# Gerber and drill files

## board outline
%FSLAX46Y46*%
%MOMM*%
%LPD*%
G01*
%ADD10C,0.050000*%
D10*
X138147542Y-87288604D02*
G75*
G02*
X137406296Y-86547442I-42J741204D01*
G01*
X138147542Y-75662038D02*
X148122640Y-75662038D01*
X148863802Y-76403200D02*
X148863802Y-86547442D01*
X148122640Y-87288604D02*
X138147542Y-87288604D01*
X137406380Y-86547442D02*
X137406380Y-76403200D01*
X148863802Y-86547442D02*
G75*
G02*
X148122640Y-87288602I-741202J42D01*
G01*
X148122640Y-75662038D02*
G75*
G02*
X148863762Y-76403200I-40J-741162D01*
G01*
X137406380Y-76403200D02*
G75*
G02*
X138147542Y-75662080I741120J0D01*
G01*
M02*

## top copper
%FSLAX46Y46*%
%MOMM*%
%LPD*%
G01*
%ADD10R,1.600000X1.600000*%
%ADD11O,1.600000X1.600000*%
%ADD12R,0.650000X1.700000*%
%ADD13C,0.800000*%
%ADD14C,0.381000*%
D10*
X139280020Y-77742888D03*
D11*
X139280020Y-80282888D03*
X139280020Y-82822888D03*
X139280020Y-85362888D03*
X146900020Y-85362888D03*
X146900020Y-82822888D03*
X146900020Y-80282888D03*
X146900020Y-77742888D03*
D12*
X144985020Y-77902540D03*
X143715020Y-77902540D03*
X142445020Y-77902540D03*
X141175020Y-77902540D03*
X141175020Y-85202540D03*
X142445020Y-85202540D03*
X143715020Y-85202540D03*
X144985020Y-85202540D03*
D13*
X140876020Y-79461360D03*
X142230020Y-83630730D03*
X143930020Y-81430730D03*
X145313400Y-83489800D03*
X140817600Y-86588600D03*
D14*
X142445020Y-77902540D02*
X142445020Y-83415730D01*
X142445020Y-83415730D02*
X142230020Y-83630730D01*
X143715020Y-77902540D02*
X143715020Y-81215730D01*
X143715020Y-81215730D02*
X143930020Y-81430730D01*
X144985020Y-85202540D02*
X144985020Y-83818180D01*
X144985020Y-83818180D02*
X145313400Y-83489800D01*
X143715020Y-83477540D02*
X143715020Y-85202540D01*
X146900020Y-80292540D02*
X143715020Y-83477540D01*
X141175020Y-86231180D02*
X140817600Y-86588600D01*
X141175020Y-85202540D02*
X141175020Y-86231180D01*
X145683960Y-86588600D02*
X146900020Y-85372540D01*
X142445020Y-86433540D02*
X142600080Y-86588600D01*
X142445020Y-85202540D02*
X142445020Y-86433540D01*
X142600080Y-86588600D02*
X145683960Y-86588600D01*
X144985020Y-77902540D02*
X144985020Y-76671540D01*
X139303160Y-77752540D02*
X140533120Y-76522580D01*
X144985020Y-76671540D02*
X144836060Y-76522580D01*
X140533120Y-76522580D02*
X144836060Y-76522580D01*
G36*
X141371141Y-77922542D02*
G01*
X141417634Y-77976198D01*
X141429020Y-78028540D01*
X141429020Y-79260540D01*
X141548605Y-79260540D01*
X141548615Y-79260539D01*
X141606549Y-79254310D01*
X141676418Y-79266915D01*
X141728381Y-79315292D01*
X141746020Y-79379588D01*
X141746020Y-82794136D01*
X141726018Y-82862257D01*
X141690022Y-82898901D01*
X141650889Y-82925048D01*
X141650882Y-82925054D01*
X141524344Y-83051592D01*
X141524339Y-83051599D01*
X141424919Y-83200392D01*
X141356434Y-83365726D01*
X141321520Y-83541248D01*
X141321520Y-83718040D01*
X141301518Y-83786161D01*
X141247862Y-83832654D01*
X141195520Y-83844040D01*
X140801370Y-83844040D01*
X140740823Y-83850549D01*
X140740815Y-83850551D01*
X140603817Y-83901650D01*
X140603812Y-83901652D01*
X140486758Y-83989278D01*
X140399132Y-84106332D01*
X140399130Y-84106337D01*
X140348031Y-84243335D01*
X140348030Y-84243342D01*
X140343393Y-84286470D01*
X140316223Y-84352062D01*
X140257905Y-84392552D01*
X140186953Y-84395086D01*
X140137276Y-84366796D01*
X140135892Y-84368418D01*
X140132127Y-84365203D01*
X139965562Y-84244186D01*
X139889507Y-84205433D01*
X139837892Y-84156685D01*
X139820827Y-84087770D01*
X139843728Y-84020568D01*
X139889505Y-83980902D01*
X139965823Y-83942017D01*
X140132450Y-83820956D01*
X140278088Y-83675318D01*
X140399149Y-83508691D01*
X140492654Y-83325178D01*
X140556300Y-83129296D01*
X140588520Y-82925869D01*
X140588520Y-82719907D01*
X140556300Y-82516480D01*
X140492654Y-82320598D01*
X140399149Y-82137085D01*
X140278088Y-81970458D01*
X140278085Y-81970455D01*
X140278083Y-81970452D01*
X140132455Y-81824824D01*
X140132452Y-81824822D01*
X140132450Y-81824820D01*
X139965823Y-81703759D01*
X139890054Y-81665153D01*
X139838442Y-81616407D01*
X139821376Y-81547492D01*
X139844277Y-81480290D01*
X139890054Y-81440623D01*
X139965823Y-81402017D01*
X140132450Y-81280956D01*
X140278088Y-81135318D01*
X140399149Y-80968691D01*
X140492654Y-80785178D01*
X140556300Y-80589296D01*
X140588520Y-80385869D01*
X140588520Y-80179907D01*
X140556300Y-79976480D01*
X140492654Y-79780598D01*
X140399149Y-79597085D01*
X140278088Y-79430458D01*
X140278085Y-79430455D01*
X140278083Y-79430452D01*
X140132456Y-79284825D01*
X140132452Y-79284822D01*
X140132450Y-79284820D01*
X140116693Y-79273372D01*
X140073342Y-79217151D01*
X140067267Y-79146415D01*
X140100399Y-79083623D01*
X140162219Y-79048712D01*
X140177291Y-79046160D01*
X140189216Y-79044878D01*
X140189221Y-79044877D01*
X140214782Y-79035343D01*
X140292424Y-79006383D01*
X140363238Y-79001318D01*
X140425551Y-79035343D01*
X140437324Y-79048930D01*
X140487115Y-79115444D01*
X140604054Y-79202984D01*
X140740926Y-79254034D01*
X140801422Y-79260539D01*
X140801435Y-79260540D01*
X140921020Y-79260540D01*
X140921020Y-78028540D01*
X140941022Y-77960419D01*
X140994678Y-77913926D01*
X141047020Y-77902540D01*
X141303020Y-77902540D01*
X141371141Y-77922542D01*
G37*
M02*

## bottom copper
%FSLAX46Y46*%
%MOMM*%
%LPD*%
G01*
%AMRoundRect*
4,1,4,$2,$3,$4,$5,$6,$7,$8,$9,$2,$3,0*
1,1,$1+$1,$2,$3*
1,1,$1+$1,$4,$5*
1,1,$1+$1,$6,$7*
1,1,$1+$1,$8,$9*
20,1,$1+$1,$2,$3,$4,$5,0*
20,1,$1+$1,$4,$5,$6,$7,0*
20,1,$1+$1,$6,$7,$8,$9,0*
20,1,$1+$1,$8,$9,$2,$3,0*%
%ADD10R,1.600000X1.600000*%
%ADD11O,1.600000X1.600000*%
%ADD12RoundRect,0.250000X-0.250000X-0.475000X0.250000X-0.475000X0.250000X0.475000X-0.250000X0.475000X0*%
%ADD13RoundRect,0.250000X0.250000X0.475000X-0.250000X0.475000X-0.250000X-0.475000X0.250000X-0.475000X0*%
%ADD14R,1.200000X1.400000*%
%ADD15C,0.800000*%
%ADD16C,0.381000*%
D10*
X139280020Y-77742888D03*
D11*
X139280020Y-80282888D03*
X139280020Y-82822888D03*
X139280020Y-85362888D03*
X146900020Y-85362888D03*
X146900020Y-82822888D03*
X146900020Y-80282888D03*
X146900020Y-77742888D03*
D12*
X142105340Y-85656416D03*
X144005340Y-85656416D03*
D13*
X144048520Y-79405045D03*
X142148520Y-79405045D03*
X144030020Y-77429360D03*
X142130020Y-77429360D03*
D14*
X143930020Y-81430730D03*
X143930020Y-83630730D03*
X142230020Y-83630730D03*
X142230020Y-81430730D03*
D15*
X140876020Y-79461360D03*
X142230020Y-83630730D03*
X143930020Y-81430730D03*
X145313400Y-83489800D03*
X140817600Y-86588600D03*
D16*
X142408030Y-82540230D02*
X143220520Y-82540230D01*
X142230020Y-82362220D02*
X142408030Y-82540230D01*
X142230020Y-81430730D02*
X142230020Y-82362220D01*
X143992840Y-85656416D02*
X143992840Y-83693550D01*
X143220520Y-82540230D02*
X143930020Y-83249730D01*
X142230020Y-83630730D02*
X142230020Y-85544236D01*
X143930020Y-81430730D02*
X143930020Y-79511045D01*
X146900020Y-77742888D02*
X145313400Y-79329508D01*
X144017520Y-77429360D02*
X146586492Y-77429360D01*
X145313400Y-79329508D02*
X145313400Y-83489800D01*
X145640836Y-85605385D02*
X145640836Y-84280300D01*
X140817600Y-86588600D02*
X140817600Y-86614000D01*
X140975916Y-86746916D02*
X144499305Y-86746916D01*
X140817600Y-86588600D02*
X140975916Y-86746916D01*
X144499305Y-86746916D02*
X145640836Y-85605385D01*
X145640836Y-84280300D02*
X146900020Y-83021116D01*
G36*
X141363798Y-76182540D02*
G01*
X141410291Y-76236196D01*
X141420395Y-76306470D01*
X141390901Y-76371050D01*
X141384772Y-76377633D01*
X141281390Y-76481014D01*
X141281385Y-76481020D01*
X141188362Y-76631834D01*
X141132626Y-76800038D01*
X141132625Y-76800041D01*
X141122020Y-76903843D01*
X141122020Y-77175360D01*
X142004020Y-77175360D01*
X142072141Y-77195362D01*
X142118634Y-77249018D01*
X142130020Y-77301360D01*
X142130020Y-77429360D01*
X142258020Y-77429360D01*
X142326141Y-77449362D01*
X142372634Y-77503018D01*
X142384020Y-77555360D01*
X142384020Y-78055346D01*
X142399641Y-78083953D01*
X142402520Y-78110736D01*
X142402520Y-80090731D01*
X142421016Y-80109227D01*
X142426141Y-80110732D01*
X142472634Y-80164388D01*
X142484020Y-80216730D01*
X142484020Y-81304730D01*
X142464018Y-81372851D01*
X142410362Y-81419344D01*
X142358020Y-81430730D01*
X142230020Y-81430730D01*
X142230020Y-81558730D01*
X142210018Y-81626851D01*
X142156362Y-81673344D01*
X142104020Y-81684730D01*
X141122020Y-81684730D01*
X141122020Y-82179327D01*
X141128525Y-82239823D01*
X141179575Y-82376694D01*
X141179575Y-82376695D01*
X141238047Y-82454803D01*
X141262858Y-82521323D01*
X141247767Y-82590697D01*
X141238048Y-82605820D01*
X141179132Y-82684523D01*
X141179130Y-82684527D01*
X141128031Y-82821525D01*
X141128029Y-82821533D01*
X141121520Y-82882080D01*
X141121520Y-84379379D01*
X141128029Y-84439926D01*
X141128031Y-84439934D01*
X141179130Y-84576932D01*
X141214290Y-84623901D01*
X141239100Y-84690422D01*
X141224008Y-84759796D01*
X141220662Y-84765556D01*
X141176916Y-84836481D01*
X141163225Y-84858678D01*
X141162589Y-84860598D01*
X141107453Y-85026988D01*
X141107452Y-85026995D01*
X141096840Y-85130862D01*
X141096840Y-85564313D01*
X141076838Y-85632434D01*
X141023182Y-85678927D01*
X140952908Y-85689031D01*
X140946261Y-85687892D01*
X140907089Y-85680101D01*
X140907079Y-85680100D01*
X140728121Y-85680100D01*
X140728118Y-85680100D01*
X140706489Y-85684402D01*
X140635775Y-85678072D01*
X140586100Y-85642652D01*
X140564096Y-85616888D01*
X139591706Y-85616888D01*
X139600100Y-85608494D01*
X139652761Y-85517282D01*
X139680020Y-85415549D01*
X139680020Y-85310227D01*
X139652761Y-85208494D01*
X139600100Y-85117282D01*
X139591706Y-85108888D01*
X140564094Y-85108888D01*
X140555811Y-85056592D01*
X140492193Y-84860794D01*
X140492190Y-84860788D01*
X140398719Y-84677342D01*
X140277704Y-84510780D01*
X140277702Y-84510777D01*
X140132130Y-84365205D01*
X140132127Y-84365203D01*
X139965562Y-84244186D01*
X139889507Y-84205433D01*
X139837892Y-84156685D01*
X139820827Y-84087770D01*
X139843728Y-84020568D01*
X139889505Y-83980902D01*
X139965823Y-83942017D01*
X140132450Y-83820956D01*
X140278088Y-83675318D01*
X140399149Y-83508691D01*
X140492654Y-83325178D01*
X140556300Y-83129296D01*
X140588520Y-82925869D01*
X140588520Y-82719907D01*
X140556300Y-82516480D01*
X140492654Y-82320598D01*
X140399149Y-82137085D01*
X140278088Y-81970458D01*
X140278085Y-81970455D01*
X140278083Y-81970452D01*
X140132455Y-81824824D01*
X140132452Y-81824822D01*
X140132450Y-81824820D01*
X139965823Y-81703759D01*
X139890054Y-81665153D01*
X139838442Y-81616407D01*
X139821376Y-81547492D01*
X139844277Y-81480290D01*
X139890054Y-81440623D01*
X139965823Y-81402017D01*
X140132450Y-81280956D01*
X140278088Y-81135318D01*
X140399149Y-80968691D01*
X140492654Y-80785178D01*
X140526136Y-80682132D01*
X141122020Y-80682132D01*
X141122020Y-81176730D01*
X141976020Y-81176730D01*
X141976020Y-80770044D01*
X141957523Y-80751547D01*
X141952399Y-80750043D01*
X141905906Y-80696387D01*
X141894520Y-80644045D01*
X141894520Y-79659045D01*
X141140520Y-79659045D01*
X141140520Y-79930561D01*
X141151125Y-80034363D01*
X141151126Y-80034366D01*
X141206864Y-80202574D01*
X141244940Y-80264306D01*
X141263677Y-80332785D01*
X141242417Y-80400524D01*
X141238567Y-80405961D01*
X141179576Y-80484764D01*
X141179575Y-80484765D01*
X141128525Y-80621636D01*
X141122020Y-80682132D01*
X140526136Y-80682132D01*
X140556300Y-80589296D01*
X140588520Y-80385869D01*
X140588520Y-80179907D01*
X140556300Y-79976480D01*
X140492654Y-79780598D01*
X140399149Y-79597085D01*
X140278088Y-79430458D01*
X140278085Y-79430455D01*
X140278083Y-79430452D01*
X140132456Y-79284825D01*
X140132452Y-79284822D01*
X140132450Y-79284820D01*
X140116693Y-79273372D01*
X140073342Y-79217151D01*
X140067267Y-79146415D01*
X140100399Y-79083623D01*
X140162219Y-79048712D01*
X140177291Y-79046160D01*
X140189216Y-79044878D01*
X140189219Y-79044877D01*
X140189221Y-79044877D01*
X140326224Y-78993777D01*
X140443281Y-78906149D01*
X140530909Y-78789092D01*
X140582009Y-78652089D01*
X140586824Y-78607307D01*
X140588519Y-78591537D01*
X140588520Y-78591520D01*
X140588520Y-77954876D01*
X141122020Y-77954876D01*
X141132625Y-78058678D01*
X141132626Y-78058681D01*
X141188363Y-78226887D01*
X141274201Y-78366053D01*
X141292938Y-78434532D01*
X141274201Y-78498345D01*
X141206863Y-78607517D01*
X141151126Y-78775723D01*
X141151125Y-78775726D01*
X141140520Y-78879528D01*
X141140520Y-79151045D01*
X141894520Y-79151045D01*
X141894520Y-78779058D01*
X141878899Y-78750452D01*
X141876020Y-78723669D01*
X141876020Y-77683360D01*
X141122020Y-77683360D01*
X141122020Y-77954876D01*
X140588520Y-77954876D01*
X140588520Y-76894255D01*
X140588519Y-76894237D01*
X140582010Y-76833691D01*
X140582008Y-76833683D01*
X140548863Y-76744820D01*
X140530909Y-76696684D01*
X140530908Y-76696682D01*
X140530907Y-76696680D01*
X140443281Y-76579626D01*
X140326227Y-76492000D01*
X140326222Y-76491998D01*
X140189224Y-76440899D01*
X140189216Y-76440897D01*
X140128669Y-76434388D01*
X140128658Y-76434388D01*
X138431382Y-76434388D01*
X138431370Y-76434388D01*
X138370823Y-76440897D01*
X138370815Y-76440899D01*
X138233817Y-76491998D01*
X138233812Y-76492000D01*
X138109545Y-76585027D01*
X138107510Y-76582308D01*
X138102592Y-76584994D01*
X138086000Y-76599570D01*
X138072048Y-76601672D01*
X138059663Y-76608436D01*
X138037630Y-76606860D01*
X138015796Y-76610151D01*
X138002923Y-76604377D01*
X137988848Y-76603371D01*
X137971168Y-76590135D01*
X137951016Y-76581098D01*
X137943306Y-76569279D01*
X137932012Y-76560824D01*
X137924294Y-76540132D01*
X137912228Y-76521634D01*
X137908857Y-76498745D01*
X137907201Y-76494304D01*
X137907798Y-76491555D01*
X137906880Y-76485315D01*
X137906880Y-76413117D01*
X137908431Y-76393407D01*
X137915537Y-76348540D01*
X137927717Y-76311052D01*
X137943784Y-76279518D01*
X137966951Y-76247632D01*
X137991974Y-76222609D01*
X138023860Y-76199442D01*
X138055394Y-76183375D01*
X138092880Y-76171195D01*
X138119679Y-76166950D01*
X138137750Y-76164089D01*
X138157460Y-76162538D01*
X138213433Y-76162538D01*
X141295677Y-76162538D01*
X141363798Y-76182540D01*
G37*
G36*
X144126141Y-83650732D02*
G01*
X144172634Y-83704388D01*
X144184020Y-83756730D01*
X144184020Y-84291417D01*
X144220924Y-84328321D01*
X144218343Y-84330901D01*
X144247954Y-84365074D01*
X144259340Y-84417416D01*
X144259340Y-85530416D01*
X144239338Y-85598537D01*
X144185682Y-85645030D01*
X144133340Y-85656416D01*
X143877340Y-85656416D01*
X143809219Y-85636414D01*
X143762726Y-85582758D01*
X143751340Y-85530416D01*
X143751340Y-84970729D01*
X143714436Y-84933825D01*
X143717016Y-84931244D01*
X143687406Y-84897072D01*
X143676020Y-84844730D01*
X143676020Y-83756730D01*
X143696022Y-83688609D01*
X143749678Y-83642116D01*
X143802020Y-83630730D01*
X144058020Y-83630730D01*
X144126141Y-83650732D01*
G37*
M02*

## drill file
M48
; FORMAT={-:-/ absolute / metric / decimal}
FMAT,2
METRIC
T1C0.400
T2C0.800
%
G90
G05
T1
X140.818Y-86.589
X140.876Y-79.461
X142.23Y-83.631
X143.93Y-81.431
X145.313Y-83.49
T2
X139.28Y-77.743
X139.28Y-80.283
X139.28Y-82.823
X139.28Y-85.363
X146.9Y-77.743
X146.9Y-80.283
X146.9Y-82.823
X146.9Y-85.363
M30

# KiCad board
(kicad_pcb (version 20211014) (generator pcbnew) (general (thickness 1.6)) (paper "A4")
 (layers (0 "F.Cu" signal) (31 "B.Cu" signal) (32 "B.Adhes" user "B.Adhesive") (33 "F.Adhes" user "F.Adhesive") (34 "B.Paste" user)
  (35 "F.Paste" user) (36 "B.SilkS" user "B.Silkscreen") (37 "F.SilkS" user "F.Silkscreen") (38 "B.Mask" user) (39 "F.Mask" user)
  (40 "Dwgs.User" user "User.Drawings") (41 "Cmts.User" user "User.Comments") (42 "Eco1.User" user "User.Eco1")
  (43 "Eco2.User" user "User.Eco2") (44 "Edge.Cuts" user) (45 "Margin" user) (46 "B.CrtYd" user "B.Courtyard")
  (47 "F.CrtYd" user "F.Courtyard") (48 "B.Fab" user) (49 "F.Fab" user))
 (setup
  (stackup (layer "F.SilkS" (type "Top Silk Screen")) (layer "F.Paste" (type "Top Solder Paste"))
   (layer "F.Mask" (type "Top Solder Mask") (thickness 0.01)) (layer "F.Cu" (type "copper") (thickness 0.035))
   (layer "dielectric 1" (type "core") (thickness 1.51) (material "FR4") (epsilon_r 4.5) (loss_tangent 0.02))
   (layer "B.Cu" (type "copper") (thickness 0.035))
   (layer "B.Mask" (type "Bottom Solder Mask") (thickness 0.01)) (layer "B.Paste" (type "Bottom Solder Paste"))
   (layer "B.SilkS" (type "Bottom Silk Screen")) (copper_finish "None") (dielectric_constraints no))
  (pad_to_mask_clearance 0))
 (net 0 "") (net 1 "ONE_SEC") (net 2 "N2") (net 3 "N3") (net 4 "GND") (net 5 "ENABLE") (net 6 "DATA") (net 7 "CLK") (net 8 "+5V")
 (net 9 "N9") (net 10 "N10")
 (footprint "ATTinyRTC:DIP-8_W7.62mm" (layer "F.Cu") (at 139.28002 77.742888)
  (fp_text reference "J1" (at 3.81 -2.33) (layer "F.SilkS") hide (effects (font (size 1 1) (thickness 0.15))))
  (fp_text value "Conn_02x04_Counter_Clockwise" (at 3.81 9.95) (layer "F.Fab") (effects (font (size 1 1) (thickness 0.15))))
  (pad "1" thru_hole rect (at 0 0) (size 1.6 1.6) (drill 0.8) (layers *.Cu *.Mask) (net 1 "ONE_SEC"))
  (pad "2" thru_hole oval (at 0 2.54) (size 1.6 1.6) (drill 0.8) (layers *.Cu *.Mask) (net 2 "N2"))
  (pad "3" thru_hole oval (at 0 5.08) (size 1.6 1.6) (drill 0.8) (layers *.Cu *.Mask) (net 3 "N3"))
  (pad "4" thru_hole oval (at 0 7.62) (size 1.6 1.6) (drill 0.8) (layers *.Cu *.Mask) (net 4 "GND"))
  (pad "5" thru_hole oval (at 7.62 7.62) (size 1.6 1.6) (drill 0.8) (layers *.Cu *.Mask) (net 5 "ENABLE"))
  (pad "6" thru_hole oval (at 7.62 5.08) (size 1.6 1.6) (drill 0.8) (layers *.Cu *.Mask) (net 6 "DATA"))
  (pad "7" thru_hole oval (at 7.62 2.54) (size 1.6 1.6) (drill 0.8) (layers *.Cu *.Mask) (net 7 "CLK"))
  (pad "8" thru_hole oval (at 7.62 0) (size 1.6 1.6) (drill 0.8) (layers *.Cu *.Mask) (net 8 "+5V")))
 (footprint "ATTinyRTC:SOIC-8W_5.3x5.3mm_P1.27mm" (layer "F.Cu") (at 143.08002 81.55254 -90)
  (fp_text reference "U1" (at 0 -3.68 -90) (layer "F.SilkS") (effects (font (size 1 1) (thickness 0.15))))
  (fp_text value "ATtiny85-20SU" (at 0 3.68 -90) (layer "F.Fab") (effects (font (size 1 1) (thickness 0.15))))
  (pad "1" smd rect (at -3.65 -1.905 270) (size 1.7 0.65) (layers "F.Cu" "F.Paste" "F.Mask") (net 1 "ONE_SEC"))
  (pad "2" smd rect (at -3.65 -0.635 270) (size 1.7 0.65) (layers "F.Cu" "F.Paste" "F.Mask") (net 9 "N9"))
  (pad "3" smd rect (at -3.65 0.635 270) (size 1.7 0.65) (layers "F.Cu" "F.Paste" "F.Mask") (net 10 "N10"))
  (pad "4" smd rect (at -3.65 1.905 270) (size 1.7 0.65) (layers "F.Cu" "F.Paste" "F.Mask") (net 4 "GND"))
  (pad "5" smd rect (at 3.65 1.905 270) (size 1.7 0.65) (layers "F.Cu" "F.Paste" "F.Mask") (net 6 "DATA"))
  (pad "6" smd rect (at 3.65 0.635 270) (size 1.7 0.65) (layers "F.Cu" "F.Paste" "F.Mask") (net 5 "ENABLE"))
  (pad "7" smd rect (at 3.65 -0.635 270) (size 1.7 0.65) (layers "F.Cu" "F.Paste" "F.Mask") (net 7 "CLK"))
  (pad "8" smd rect (at 3.65 -1.905 270) (size 1.7 0.65) (layers "F.Cu" "F.Paste" "F.Mask") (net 8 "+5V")))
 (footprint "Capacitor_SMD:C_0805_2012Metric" (layer "B.Cu") (at 143.05534 85.656416)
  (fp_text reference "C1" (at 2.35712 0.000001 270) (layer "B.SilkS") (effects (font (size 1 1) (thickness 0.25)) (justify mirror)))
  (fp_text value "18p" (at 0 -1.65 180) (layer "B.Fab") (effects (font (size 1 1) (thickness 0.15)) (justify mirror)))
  (pad "1" smd roundrect (at -0.95 0) (size 1 1.45) (layers "B.Cu" "B.Paste" "B.Mask") (roundrect_rratio 0.25) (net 10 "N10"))
  (pad "2" smd roundrect (at 0.95 0) (size 1 1.45) (layers "B.Cu" "B.Paste" "B.Mask") (roundrect_rratio 0.25) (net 4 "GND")))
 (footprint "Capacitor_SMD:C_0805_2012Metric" (layer "B.Cu") (at 143.09852 79.405045 180)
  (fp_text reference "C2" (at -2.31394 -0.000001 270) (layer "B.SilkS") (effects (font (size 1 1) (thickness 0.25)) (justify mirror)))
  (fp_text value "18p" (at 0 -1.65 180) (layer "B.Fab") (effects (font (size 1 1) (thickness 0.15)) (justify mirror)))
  (pad "1" smd roundrect (at -0.95 0 180) (size 1 1.45) (layers "B.Cu" "B.Paste" "B.Mask") (roundrect_rratio 0.25) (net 9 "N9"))
  (pad "2" smd roundrect (at 0.95 0 180) (size 1 1.45) (layers "B.Cu" "B.Paste" "B.Mask") (roundrect_rratio 0.25) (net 4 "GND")))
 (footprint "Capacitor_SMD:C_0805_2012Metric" (layer "B.Cu") (at 143.08002 77.42936 180)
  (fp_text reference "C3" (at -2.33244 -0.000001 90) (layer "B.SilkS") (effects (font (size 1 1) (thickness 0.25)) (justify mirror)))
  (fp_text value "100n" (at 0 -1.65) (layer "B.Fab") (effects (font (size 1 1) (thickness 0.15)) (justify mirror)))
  (pad "1" smd roundrect (at -0.95 0 180) (size 1 1.45) (layers "B.Cu" "B.Paste" "B.Mask") (roundrect_rratio 0.25) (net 8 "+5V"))
  (pad "2" smd roundrect (at 0.95 0 180) (size 1 1.45) (layers "B.Cu" "B.Paste" "B.Mask") (roundrect_rratio 0.25) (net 4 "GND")))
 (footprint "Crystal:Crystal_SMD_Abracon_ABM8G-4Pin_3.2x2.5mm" (layer "B.Cu") (at 143.08002 82.53073 -90)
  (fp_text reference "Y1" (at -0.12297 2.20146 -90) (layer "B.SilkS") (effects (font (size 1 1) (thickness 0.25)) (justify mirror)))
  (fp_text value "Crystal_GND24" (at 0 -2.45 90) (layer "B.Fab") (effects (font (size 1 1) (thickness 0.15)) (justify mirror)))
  (pad "1" smd rect (at -1.1 -0.85 270) (size 1.4 1.2) (layers "B.Cu" "B.Paste" "B.Mask") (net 9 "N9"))
  (pad "2" smd rect (at 1.1 -0.85 270) (size 1.4 1.2) (layers "B.Cu" "B.Paste" "B.Mask") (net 4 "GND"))
  (pad "3" smd rect (at 1.1 0.85 270) (size 1.4 1.2) (layers "B.Cu" "B.Paste" "B.Mask") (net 10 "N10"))
  (pad "4" smd rect (at -1.1 0.85 270) (size 1.4 1.2) (layers "B.Cu" "B.Paste" "B.Mask") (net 4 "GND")))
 (gr_arc (start 138.147542 87.288604) (mid 137.623461 87.071523) (end 137.40638 86.547442) (layer "Edge.Cuts") (width 0.05))
 (gr_line (start 138.147542 75.662038) (end 148.12264 75.662038) (layer "Edge.Cuts") (width 0.05))
 (gr_line (start 148.863802 76.4032) (end 148.863802 86.547442) (layer "Edge.Cuts") (width 0.05))
 (gr_line (start 148.12264 87.288604) (end 138.147542 87.288604) (layer "Edge.Cuts") (width 0.05))
 (gr_line (start 137.40638 86.547442) (end 137.40638 76.4032) (layer "Edge.Cuts") (width 0.05))
 (gr_arc (start 148.863802 86.547442) (mid 148.646721 87.071523) (end 148.12264 87.288604) (layer "Edge.Cuts") (width 0.05))
 (gr_arc (start 148.12264 75.662038) (mid 148.646721 75.879119) (end 148.863802 76.4032) (layer "Edge.Cuts") (width 0.05))
 (gr_arc (start 137.40638 76.4032) (mid 137.623461 75.879119) (end 138.147542 75.662038) (layer "Edge.Cuts") (width 0.05))
 (via (at 140.87602 79.46136) (size 0.8) (drill 0.4) (layers "F.Cu" "B.Cu") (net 4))
 (segment (start 142.40803 82.54023) (end 143.22052 82.54023) (width 0.381) (layer "B.Cu") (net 4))
 (segment (start 142.23002 82.36222) (end 142.40803 82.54023) (width 0.381) (layer "B.Cu") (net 4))
 (segment (start 142.23002 81.43073) (end 142.23002 82.36222) (width 0.381) (layer "B.Cu") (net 4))
 (segment (start 143.99284 85.656416) (end 143.99284 83.69355) (width 0.381) (layer "B.Cu") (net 4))
 (segment (start 143.22052 82.54023) (end 143.93002 83.24973) (width 0.381) (layer "B.Cu") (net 4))
 (segment (start 142.44502 77.90254) (end 142.44502 83.41573) (width 0.381) (layer "F.Cu") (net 10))
 (segment (start 142.44502 83.41573) (end 142.23002 83.63073) (width 0.381) (layer "F.Cu") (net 10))
 (via (at 142.23002 83.63073) (size 0.8) (drill 0.4) (layers "F.Cu" "B.Cu") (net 10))
 (segment (start 142.23002 83.63073) (end 142.23002 85.544236) (width 0.381) (layer "B.Cu") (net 10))
 (segment (start 143.71502 77.90254) (end 143.71502 81.21573) (width 0.381) (layer "F.Cu") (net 9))
 (segment (start 143.71502 81.21573) (end 143.93002 81.43073) (width 0.381) (layer "F.Cu") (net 9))
 (via (at 143.93002 81.43073) (size 0.8) (drill 0.4) (layers "F.Cu" "B.Cu") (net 9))
 (segment (start 143.93002 81.43073) (end 143.93002 79.511045) (width 0.381) (layer "B.Cu") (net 9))
 (segment (start 144.98502 85.20254) (end 144.98502 83.81818) (width 0.381) (layer "F.Cu") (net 8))
 (segment (start 144.98502 83.81818) (end 145.3134 83.4898) (width 0.381) (layer "F.Cu") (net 8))
 (via (at 145.3134 83.4898) (size 0.8) (drill 0.4) (layers "F.Cu" "B.Cu") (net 8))
 (segment (start 146.90002 77.742888) (end 145.3134 79.329508) (width 0.381) (layer "B.Cu") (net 8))
 (segment (start 144.01752 77.42936) (end 146.586492 77.42936) (width 0.381) (layer "B.Cu") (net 8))
 (segment (start 145.3134 79.329508) (end 145.3134 83.4898) (width 0.381) (layer "B.Cu") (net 8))
 (segment (start 143.71502 83.47754) (end 143.71502 85.20254) (width 0.381) (layer "F.Cu") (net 7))
 (segment (start 146.90002 80.29254) (end 143.71502 83.47754) (width 0.381) (layer "F.Cu") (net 7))
 (segment (start 141.17502 86.23118) (end 140.8176 86.5886) (width 0.381) (layer "F.Cu") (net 6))
 (segment (start 141.17502 85.20254) (end 141.17502 86.23118) (width 0.381) (layer "F.Cu") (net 6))
 (via (at 140.8176 86.5886) (size 0.8) (drill 0.4) (layers "F.Cu" "B.Cu") (free) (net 6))
 (segment (start 145.640836 85.605385) (end 145.640836 84.2803) (width 0.381) (layer "B.Cu") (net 6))
 (segment (start 140.8176 86.5886) (end 140.8176 86.614) (width 0.381) (layer "B.Cu") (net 6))
 (segment (start 140.975916 86.746916) (end 144.499305 86.746916) (width 0.381) (layer "B.Cu") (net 6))
 (segment (start 140.8176 86.5886) (end 140.975916 86.746916) (width 0.381) (layer "B.Cu") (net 6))
 (segment (start 144.499305 86.746916) (end 145.640836 85.605385) (width 0.381) (layer "B.Cu") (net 6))
 (segment (start 145.640836 84.2803) (end 146.90002 83.021116) (width 0.381) (layer "B.Cu") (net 6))
 (segment (start 145.68396 86.5886) (end 146.90002 85.37254) (width 0.381) (layer "F.Cu") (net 5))
 (segment (start 142.44502 86.43354) (end 142.60008 86.5886) (width 0.381) (layer "F.Cu") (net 5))
 (segment (start 142.44502 85.20254) (end 142.44502 86.43354) (width 0.381) (layer "F.Cu") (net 5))
 (segment (start 142.60008 86.5886) (end 145.68396 86.5886) (width 0.381) (layer "F.Cu") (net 5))
 (segment (start 144.98502 77.90254) (end 144.98502 76.67154) (width 0.381) (layer "F.Cu") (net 1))
 (segment (start 139.30316 77.75254) (end 140.53312 76.52258) (width 0.381) (layer "F.Cu") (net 1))
 (segment (start 144.98502 76.67154) (end 144.83606 76.52258) (width 0.381) (layer "F.Cu") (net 1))
 (segment (start 140.53312 76.52258) (end 144.83606 76.52258) (width 0.381) (layer "F.Cu") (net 1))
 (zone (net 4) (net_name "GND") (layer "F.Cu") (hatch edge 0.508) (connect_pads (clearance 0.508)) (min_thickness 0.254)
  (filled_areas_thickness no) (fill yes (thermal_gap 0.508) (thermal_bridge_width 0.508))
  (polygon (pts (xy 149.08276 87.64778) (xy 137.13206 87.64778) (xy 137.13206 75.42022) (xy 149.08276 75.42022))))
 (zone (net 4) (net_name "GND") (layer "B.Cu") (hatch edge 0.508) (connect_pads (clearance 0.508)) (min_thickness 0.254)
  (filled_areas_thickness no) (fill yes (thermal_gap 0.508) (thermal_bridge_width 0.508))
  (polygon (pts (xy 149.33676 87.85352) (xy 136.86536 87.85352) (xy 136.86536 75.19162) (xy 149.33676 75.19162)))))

